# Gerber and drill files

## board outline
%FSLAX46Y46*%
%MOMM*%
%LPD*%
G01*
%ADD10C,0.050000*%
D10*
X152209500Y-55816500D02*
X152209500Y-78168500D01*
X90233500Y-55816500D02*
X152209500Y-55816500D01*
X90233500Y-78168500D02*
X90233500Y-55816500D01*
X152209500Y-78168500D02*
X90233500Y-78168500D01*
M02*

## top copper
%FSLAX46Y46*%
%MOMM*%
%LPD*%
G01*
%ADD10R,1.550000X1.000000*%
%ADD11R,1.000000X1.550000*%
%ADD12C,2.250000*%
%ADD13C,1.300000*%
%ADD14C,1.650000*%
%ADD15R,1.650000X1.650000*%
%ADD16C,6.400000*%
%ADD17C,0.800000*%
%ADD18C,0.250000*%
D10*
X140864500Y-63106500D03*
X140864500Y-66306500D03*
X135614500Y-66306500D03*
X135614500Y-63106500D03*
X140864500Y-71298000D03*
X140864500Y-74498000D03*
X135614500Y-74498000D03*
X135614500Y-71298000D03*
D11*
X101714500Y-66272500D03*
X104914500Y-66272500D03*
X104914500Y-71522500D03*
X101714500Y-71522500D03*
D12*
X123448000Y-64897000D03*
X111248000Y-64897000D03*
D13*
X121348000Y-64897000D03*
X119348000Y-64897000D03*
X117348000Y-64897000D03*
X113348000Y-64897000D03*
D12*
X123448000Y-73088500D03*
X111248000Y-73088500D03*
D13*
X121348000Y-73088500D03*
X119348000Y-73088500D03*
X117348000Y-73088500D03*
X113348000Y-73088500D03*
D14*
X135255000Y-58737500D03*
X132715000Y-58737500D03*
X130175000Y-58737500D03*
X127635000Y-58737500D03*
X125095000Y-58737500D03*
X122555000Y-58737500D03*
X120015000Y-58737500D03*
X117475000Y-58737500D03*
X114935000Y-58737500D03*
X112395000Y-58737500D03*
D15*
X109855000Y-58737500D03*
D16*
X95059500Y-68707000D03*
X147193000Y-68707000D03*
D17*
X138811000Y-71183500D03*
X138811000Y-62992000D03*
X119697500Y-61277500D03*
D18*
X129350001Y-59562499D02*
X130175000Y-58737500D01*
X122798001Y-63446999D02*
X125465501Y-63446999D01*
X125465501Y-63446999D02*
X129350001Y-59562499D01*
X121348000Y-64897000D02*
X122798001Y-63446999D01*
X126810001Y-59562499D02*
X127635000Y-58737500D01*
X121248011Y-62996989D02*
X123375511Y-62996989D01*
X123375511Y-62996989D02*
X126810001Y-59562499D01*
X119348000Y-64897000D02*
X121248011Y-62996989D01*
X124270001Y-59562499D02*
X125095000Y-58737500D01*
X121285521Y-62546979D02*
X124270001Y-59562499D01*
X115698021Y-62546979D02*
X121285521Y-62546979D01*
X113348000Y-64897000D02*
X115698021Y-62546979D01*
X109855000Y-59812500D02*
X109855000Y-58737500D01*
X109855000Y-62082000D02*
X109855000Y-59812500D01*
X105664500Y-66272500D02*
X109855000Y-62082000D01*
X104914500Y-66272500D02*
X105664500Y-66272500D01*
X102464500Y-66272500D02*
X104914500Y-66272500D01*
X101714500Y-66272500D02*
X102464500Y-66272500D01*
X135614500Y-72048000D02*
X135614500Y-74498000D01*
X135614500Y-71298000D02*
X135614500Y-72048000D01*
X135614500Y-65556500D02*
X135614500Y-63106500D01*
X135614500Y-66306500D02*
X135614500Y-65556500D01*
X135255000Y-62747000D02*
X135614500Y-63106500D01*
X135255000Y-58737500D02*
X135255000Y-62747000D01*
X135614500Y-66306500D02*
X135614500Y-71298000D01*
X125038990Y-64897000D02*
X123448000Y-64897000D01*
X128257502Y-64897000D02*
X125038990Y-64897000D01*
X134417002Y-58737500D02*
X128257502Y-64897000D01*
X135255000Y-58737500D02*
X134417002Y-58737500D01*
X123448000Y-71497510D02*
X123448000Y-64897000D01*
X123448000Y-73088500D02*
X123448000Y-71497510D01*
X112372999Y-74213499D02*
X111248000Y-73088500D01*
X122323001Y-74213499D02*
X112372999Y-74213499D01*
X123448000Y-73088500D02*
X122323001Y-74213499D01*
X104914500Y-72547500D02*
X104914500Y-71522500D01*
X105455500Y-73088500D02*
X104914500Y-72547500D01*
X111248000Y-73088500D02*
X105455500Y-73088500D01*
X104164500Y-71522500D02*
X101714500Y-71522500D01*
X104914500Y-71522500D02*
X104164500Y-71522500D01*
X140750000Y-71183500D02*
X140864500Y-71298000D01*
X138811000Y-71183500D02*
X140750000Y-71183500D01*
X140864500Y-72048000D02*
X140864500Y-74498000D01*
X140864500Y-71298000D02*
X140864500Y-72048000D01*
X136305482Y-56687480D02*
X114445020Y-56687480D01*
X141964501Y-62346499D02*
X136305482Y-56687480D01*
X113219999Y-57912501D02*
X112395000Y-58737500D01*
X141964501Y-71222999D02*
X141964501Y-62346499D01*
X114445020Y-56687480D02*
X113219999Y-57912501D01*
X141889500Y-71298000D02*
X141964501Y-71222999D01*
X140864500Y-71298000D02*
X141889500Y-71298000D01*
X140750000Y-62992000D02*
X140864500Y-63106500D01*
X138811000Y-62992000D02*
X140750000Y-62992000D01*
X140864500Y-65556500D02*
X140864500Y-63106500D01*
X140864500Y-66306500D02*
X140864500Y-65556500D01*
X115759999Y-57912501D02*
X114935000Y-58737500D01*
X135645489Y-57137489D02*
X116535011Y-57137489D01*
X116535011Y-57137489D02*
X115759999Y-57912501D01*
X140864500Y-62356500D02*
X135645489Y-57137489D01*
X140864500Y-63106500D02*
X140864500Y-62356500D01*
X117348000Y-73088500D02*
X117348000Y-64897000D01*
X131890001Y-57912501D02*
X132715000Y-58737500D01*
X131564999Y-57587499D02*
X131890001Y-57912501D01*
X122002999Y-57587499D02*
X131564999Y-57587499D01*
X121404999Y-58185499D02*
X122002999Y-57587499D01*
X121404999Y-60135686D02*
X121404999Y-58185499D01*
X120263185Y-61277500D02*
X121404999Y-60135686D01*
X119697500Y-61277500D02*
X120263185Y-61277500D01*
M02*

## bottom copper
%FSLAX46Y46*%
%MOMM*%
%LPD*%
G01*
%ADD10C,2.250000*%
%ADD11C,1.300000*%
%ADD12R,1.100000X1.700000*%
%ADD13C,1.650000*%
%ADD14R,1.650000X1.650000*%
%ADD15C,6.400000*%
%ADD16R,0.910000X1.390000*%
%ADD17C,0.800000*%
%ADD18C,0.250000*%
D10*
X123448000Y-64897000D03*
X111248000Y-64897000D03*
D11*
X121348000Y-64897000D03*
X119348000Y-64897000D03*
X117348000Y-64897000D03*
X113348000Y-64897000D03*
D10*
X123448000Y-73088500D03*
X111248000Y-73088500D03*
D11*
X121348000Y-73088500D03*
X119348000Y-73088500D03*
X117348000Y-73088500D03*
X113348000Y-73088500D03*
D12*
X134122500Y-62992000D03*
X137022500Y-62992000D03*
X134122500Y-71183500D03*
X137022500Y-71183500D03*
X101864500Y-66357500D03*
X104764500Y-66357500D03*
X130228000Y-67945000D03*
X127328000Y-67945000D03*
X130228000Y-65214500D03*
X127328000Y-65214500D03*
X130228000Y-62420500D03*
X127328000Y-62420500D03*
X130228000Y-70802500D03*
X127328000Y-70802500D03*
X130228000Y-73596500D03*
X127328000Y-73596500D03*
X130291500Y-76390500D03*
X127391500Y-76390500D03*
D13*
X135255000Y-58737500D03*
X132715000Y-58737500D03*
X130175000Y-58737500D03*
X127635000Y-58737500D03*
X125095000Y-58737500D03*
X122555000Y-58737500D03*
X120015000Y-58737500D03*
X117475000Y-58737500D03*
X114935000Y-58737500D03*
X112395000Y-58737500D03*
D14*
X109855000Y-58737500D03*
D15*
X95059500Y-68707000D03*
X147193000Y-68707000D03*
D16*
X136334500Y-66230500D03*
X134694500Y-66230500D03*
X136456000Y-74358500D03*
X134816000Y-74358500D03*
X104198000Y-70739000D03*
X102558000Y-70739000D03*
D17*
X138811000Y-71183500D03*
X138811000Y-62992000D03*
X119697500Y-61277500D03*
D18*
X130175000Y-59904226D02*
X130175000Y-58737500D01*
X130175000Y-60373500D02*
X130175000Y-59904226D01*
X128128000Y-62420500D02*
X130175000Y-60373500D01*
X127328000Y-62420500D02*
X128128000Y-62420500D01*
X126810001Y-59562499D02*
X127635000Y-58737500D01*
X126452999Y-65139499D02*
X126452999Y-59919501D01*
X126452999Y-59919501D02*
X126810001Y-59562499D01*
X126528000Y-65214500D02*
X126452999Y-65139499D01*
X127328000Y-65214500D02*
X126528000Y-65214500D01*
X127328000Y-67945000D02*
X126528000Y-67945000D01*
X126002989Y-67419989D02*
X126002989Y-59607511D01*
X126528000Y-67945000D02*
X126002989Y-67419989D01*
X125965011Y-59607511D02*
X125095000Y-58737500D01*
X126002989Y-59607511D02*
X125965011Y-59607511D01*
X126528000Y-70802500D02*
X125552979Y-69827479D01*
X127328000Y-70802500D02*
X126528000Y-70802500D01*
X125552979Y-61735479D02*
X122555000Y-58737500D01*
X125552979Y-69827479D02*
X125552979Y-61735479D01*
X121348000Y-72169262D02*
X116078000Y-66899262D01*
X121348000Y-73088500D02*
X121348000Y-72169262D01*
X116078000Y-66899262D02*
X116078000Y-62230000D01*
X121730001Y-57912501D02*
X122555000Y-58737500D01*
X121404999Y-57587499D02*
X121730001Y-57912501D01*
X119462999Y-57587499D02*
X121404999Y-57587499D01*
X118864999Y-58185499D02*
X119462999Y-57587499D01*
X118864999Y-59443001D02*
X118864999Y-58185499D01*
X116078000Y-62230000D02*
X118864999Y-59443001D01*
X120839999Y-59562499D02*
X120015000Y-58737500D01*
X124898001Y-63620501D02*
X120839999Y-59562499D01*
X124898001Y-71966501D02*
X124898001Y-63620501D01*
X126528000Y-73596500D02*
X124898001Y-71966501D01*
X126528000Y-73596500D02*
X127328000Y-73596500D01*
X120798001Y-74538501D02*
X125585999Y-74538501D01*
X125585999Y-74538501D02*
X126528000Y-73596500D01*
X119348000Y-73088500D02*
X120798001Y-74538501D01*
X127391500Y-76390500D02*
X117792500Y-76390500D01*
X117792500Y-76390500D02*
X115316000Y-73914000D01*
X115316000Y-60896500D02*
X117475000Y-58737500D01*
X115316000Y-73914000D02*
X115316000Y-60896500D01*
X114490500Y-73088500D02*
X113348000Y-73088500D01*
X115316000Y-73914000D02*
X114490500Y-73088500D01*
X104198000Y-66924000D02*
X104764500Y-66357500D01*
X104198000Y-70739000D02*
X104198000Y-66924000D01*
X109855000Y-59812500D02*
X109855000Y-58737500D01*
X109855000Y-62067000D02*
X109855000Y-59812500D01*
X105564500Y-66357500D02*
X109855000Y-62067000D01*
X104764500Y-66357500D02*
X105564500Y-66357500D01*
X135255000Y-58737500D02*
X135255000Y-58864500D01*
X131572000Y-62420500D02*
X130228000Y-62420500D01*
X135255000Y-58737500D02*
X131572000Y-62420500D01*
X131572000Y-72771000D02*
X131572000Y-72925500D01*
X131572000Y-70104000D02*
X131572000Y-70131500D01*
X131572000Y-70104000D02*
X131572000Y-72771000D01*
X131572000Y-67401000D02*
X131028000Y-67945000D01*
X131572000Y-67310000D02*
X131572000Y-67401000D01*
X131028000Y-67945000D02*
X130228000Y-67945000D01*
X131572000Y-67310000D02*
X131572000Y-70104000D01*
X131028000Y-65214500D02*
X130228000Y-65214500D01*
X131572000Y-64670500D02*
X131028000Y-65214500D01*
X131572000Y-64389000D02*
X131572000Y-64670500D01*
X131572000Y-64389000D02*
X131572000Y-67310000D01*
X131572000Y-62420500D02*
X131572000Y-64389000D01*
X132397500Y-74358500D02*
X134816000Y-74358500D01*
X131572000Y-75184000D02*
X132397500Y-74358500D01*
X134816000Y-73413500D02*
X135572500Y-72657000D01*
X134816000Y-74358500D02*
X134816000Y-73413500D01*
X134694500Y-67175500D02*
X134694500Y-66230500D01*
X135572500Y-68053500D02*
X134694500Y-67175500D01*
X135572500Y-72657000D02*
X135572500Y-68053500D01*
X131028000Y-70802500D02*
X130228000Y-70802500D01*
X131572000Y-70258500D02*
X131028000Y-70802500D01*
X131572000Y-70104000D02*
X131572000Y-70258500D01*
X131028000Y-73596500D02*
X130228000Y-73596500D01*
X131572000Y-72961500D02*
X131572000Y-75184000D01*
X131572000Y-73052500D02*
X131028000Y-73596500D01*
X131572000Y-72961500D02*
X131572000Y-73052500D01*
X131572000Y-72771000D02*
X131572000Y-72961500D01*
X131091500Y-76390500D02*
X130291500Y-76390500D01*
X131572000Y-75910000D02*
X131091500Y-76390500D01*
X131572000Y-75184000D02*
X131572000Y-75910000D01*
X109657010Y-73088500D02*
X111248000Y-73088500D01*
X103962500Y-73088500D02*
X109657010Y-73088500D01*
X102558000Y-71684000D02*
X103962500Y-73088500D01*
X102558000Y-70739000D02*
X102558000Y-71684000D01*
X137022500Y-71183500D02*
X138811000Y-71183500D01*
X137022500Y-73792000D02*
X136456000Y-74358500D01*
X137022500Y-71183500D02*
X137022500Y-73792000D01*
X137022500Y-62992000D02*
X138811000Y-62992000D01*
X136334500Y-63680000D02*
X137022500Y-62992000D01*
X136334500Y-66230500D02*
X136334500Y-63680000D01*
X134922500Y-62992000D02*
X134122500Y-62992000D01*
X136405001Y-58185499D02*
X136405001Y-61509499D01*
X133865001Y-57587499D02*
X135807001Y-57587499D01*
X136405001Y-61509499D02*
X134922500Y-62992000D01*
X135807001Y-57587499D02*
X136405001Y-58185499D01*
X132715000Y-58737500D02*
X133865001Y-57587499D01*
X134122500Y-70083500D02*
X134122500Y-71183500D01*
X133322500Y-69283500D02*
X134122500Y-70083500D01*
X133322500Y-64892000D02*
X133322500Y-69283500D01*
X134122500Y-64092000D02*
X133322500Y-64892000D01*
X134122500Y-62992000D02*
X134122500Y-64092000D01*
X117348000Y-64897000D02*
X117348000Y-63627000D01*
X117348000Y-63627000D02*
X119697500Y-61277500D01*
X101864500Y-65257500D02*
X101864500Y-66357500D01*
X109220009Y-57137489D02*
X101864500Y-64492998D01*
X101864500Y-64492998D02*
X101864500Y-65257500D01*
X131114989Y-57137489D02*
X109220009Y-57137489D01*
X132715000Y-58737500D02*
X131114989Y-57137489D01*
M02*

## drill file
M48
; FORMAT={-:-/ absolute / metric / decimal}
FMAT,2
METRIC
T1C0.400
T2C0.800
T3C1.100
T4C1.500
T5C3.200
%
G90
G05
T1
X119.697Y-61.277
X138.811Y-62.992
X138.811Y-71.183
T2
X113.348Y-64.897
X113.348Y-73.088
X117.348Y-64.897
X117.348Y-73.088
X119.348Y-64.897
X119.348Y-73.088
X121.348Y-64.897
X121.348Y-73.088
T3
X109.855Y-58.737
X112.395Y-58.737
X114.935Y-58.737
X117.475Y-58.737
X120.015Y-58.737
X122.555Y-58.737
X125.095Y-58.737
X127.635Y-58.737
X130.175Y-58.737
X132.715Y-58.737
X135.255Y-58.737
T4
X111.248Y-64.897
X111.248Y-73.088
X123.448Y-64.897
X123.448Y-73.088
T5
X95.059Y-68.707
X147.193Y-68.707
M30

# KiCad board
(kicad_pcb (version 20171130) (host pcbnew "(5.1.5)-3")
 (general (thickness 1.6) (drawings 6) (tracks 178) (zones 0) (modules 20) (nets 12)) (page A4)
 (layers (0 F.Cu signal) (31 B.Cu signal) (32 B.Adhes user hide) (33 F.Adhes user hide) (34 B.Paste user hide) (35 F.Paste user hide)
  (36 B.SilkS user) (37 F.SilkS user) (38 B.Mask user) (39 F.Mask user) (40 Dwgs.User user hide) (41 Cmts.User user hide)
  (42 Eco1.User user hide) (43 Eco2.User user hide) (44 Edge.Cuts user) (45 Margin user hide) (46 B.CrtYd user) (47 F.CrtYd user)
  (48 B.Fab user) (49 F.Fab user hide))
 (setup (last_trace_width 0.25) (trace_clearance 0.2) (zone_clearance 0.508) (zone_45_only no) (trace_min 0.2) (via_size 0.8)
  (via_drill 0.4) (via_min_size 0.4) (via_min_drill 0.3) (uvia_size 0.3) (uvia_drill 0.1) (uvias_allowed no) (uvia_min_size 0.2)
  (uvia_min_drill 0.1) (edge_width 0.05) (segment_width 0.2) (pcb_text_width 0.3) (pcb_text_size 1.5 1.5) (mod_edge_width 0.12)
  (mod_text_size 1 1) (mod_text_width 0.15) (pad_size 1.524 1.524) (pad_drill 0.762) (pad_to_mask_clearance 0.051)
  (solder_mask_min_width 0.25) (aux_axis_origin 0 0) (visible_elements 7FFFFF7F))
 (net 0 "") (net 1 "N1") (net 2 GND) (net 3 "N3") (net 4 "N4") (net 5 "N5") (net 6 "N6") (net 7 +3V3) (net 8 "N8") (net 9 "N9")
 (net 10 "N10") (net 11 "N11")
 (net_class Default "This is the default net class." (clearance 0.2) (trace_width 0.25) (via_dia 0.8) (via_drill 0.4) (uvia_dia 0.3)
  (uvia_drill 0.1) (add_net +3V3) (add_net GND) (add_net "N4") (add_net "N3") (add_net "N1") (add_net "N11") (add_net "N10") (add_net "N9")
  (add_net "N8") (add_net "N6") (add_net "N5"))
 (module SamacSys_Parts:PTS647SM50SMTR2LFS (layer F.Cu) (at 138.2395 64.7065)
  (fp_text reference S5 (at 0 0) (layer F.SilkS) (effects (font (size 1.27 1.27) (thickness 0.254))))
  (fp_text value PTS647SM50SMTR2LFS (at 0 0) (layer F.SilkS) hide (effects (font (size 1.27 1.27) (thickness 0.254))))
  (pad 4 smd rect (at 2.625 -1.6 90) (size 1 1.55) (layers F.Cu F.Paste F.Mask) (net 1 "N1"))
  (pad 3 smd rect (at 2.625 1.6 90) (size 1 1.55) (layers F.Cu F.Paste F.Mask) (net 1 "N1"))
  (pad 2 smd rect (at -2.625 1.6 90) (size 1 1.55) (layers F.Cu F.Paste F.Mask) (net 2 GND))
  (pad 1 smd rect (at -2.625 -1.6 90) (size 1 1.55) (layers F.Cu F.Paste F.Mask) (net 2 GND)))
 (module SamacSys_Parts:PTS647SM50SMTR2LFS (layer F.Cu) (at 138.2395 72.898)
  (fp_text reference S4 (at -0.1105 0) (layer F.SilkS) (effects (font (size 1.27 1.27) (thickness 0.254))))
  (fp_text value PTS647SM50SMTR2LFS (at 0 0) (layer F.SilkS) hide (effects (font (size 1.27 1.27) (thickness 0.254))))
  (pad 4 smd rect (at 2.625 -1.6 90) (size 1 1.55) (layers F.Cu F.Paste F.Mask) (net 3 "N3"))
  (pad 3 smd rect (at 2.625 1.6 90) (size 1 1.55) (layers F.Cu F.Paste F.Mask) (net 3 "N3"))
  (pad 2 smd rect (at -2.625 1.6 90) (size 1 1.55) (layers F.Cu F.Paste F.Mask) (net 2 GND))
  (pad 1 smd rect (at -2.625 -1.6 90) (size 1 1.55) (layers F.Cu F.Paste F.Mask) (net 2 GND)))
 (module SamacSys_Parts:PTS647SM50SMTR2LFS (layer F.Cu) (at 103.3145 68.8975 90)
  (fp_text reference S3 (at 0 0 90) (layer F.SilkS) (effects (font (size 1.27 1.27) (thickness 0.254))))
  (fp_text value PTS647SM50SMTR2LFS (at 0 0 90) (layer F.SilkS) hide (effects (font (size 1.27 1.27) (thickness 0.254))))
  (pad 4 smd rect (at 2.625 -1.6 180) (size 1 1.55) (layers F.Cu F.Paste F.Mask) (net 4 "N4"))
  (pad 3 smd rect (at 2.625 1.6 180) (size 1 1.55) (layers F.Cu F.Paste F.Mask) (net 4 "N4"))
  (pad 2 smd rect (at -2.625 1.6 180) (size 1 1.55) (layers F.Cu F.Paste F.Mask) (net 2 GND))
  (pad 1 smd rect (at -2.625 -1.6 180) (size 1 1.55) (layers F.Cu F.Paste F.Mask) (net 2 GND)))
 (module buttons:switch (layer F.Cu) (at 117.348 64.897)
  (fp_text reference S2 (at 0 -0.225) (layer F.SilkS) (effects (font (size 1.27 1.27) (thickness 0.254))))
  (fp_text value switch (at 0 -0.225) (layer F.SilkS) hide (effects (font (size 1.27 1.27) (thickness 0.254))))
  (pad 6 thru_hole circle (at 6.1 0) (size 2.25 2.25) (drill 1.5) (layers *.Cu *.Mask) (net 2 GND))
  (pad 5 thru_hole circle (at -6.1 0) (size 2.25 2.25) (drill 1.5) (layers *.Cu *.Mask) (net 2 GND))
  (pad 4 thru_hole circle (at 4 0) (size 1.3 1.3) (drill 0.8) (layers *.Cu *.Mask) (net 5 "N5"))
  (pad 3 thru_hole circle (at 2 0) (size 1.3 1.3) (drill 0.8) (layers *.Cu *.Mask) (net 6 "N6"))
  (pad 2 thru_hole circle (at 0 0) (size 1.3 1.3) (drill 0.8) (layers *.Cu *.Mask) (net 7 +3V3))
  (pad 1 thru_hole circle (at -4 0) (size 1.3 1.3) (drill 0.8) (layers *.Cu *.Mask) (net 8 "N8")))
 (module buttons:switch (layer F.Cu) (at 117.348 73.0885)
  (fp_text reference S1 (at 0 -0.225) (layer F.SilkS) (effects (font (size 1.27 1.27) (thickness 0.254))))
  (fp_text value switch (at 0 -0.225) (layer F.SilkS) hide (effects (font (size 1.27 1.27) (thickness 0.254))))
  (pad 6 thru_hole circle (at 6.1 0) (size 2.25 2.25) (drill 1.5) (layers *.Cu *.Mask) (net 2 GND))
  (pad 5 thru_hole circle (at -6.1 0) (size 2.25 2.25) (drill 1.5) (layers *.Cu *.Mask) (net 2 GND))
  (pad 4 thru_hole circle (at 4 0) (size 1.3 1.3) (drill 0.8) (layers *.Cu *.Mask) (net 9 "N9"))
  (pad 3 thru_hole circle (at 2 0) (size 1.3 1.3) (drill 0.8) (layers *.Cu *.Mask) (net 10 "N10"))
  (pad 2 thru_hole circle (at 0 0) (size 1.3 1.3) (drill 0.8) (layers *.Cu *.Mask) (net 7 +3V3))
  (pad 1 thru_hole circle (at -4 0) (size 1.3 1.3) (drill 0.8) (layers *.Cu *.Mask) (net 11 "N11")))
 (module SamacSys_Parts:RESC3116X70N (layer B.Cu) (at 135.5725 62.992 180)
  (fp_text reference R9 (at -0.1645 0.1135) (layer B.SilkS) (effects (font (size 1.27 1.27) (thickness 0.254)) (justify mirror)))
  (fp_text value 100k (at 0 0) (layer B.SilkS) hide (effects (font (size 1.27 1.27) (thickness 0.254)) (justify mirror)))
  (pad 2 smd rect (at 1.45 0 180) (size 1.1 1.7) (layers B.Cu B.Paste B.Mask) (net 7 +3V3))
  (pad 1 smd rect (at -1.45 0 180) (size 1.1 1.7) (layers B.Cu B.Paste B.Mask) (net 1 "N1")))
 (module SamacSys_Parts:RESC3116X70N (layer B.Cu) (at 135.5725 71.1835 180)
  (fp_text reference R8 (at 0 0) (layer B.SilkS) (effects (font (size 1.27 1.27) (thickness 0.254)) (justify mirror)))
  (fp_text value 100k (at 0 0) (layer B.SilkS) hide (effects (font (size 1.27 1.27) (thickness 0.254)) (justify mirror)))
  (pad 2 smd rect (at 1.45 0 180) (size 1.1 1.7) (layers B.Cu B.Paste B.Mask) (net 7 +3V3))
  (pad 1 smd rect (at -1.45 0 180) (size 1.1 1.7) (layers B.Cu B.Paste B.Mask) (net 3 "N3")))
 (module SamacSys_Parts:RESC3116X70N (layer B.Cu) (at 103.3145 66.3575 180)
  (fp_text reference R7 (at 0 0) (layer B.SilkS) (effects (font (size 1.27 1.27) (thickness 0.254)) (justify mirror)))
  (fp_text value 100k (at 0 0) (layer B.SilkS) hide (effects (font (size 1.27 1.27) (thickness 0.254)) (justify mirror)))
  (pad 2 smd rect (at 1.45 0 180) (size 1.1 1.7) (layers B.Cu B.Paste B.Mask) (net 7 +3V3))
  (pad 1 smd rect (at -1.45 0 180) (size 1.1 1.7) (layers B.Cu B.Paste B.Mask) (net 4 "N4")))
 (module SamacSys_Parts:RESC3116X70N (layer B.Cu) (at 128.778 67.945)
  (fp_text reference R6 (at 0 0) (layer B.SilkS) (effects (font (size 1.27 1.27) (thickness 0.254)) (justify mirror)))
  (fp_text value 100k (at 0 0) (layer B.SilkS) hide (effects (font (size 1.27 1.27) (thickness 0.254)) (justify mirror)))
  (pad 2 smd rect (at 1.45 0) (size 1.1 1.7) (layers B.Cu B.Paste B.Mask) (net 2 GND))
  (pad 1 smd rect (at -1.45 0) (size 1.1 1.7) (layers B.Cu B.Paste B.Mask) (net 8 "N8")))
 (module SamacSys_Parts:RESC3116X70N (layer B.Cu) (at 128.778 65.2145)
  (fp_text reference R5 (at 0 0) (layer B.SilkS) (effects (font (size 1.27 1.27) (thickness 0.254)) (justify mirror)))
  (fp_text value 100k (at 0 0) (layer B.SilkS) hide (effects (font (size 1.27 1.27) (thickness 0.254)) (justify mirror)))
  (pad 2 smd rect (at 1.45 0) (size 1.1 1.7) (layers B.Cu B.Paste B.Mask) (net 2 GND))
  (pad 1 smd rect (at -1.45 0) (size 1.1 1.7) (layers B.Cu B.Paste B.Mask) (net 6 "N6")))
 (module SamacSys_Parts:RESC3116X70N (layer B.Cu) (at 128.778 62.4205)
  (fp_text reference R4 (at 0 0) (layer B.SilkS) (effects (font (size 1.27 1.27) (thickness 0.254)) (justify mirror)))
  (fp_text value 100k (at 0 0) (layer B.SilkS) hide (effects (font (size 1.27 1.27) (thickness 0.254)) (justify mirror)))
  (pad 2 smd rect (at 1.45 0) (size 1.1 1.7) (layers B.Cu B.Paste B.Mask) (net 2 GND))
  (pad 1 smd rect (at -1.45 0) (size 1.1 1.7) (layers B.Cu B.Paste B.Mask) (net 5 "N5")))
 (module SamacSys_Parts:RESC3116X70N (layer B.Cu) (at 128.778 70.8025)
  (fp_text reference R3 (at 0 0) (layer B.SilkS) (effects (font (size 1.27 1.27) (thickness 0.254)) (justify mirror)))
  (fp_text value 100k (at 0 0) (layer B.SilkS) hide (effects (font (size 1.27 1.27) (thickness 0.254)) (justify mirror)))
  (pad 2 smd rect (at 1.45 0) (size 1.1 1.7) (layers B.Cu B.Paste B.Mask) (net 2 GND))
  (pad 1 smd rect (at -1.45 0) (size 1.1 1.7) (layers B.Cu B.Paste B.Mask) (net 9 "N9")))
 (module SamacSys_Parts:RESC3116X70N (layer B.Cu) (at 128.778 73.5965)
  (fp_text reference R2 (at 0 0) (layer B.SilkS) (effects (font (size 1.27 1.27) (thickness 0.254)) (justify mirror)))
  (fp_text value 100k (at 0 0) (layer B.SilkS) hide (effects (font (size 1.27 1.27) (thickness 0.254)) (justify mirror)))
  (pad 2 smd rect (at 1.45 0) (size 1.1 1.7) (layers B.Cu B.Paste B.Mask) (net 2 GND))
  (pad 1 smd rect (at -1.45 0) (size 1.1 1.7) (layers B.Cu B.Paste B.Mask) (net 10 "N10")))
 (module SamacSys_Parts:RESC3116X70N (layer B.Cu) (at 128.8415 76.3905)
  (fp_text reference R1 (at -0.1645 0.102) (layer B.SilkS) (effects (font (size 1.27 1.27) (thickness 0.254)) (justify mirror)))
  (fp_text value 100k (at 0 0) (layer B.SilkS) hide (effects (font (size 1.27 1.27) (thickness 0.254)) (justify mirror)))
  (pad 2 smd rect (at 1.45 0) (size 1.1 1.7) (layers B.Cu B.Paste B.Mask) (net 2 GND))
  (pad 1 smd rect (at -1.45 0) (size 1.1 1.7) (layers B.Cu B.Paste B.Mask) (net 11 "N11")))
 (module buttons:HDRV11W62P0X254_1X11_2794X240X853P (layer F.Cu) (at 109.855 58.7375)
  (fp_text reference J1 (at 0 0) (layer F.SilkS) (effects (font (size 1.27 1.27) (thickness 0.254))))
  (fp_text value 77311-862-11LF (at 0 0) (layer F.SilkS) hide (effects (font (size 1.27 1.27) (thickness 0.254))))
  (pad 11 thru_hole circle (at 25.4 0) (size 1.65 1.65) (drill 1.1) (layers *.Cu *.Mask) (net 2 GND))
  (pad 10 thru_hole circle (at 22.86 0) (size 1.65 1.65) (drill 1.1) (layers *.Cu *.Mask) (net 7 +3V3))
  (pad 9 thru_hole circle (at 20.32 0) (size 1.65 1.65) (drill 1.1) (layers *.Cu *.Mask) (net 5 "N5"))
  (pad 8 thru_hole circle (at 17.78 0) (size 1.65 1.65) (drill 1.1) (layers *.Cu *.Mask) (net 6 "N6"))
  (pad 7 thru_hole circle (at 15.24 0) (size 1.65 1.65) (drill 1.1) (layers *.Cu *.Mask) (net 8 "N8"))
  (pad 6 thru_hole circle (at 12.7 0) (size 1.65 1.65) (drill 1.1) (layers *.Cu *.Mask) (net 9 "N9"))
  (pad 5 thru_hole circle (at 10.16 0) (size 1.65 1.65) (drill 1.1) (layers *.Cu *.Mask) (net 10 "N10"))
  (pad 4 thru_hole circle (at 7.62 0) (size 1.65 1.65) (drill 1.1) (layers *.Cu *.Mask) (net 11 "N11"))
  (pad 3 thru_hole circle (at 5.08 0) (size 1.65 1.65) (drill 1.1) (layers *.Cu *.Mask) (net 1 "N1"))
  (pad 2 thru_hole circle (at 2.54 0) (size 1.65 1.65) (drill 1.1) (layers *.Cu *.Mask) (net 3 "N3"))
  (pad 1 thru_hole rect (at 0 0) (size 1.65 1.65) (drill 1.1) (layers *.Cu *.Mask) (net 4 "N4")))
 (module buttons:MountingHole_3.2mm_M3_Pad (layer F.Cu) (at 95.0595 68.707)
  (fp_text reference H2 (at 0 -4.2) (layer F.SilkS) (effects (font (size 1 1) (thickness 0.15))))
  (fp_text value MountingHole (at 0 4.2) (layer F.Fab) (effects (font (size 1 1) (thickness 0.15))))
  (pad 1 thru_hole circle (at 0 0) (size 6.4 6.4) (drill 3.2) (layers *.Cu *.Mask)))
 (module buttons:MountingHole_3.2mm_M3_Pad (layer F.Cu) (at 147.193 68.707)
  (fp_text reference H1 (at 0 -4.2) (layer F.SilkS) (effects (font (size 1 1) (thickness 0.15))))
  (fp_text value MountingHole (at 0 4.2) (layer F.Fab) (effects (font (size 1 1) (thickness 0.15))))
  (pad 1 thru_hole circle (at 0 0) (size 6.4 6.4) (drill 3.2) (layers *.Cu *.Mask)))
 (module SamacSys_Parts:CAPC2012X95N (layer B.Cu) (at 135.5145 66.2305)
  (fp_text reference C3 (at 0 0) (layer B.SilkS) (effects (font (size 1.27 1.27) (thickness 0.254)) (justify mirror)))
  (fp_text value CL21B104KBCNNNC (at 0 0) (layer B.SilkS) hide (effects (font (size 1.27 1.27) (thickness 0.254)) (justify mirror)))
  (pad 2 smd rect (at 0.82 0) (size 0.91 1.39) (layers B.Cu B.Paste B.Mask) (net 1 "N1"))
  (pad 1 smd rect (at -0.82 0) (size 0.91 1.39) (layers B.Cu B.Paste B.Mask) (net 2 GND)))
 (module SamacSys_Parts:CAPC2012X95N (layer B.Cu) (at 135.636 74.3585)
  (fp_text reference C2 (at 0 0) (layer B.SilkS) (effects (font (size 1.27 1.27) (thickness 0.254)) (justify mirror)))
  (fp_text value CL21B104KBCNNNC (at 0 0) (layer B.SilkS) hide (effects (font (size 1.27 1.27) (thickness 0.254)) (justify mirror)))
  (pad 2 smd rect (at 0.82 0) (size 0.91 1.39) (layers B.Cu B.Paste B.Mask) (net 3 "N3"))
  (pad 1 smd rect (at -0.82 0) (size 0.91 1.39) (layers B.Cu B.Paste B.Mask) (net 2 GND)))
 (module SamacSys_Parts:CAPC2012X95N (layer B.Cu) (at 103.378 70.739)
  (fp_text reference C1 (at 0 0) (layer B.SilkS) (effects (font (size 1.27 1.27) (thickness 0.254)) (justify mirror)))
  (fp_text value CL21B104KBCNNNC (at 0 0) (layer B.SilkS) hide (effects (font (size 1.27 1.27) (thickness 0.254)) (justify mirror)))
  (pad 2 smd rect (at 0.82 0) (size 0.91 1.39) (layers B.Cu B.Paste B.Mask) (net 4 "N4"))
  (pad 1 smd rect (at -0.82 0) (size 0.91 1.39) (layers B.Cu B.Paste B.Mask) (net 2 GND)))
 (gr_line (start 152.2095 55.8165) (end 152.2095 78.1685) (layer Edge.Cuts) (width 0.05))
 (gr_line (start 90.2335 55.8165) (end 152.2095 55.8165) (layer Edge.Cuts) (width 0.05))
 (gr_line (start 90.2335 78.1685) (end 90.2335 55.8165) (layer Edge.Cuts) (width 0.05))
 (gr_line (start 152.2095 78.1685) (end 90.2335 78.1685) (layer Edge.Cuts) (width 0.05))
 (segment (start 130.175 59.904226) (end 130.175 58.7375) (width 0.25) (layer B.Cu) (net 5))
 (segment (start 130.175 60.3735) (end 130.175 59.904226) (width 0.25) (layer B.Cu) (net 5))
 (segment (start 128.128 62.4205) (end 130.175 60.3735) (width 0.25) (layer B.Cu) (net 5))
 (segment (start 127.328 62.4205) (end 128.128 62.4205) (width 0.25) (layer B.Cu) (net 5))
 (segment (start 129.350001 59.562499) (end 130.175 58.7375) (width 0.25) (layer F.Cu) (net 5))
 (segment (start 122.798001 63.446999) (end 125.465501 63.446999) (width 0.25) (layer F.Cu) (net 5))
 (segment (start 125.465501 63.446999) (end 129.350001 59.562499) (width 0.25) (layer F.Cu) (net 5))
 (segment (start 121.348 64.897) (end 122.798001 63.446999) (width 0.25) (layer F.Cu) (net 5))
 (segment (start 126.810001 59.562499) (end 127.635 58.7375) (width 0.25) (layer B.Cu) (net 6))
 (segment (start 126.452999 65.139499) (end 126.452999 59.919501) (width 0.25) (layer B.Cu) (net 6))
 (segment (start 126.452999 59.919501) (end 126.810001 59.562499) (width 0.25) (layer B.Cu) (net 6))
 (segment (start 126.528 65.2145) (end 126.452999 65.139499) (width 0.25) (layer B.Cu) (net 6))
 (segment (start 127.328 65.2145) (end 126.528 65.2145) (width 0.25) (layer B.Cu) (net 6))
 (segment (start 126.810001 59.562499) (end 127.635 58.7375) (width 0.25) (layer F.Cu) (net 6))
 (segment (start 121.248011 62.996989) (end 123.375511 62.996989) (width 0.25) (layer F.Cu) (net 6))
 (segment (start 123.375511 62.996989) (end 126.810001 59.562499) (width 0.25) (layer F.Cu) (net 6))
 (segment (start 119.348 64.897) (end 121.248011 62.996989) (width 0.25) (layer F.Cu) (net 6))
 (segment (start 127.328 67.945) (end 126.528 67.945) (width 0.25) (layer B.Cu) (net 8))
 (segment (start 126.002989 67.419989) (end 126.002989 59.607511) (width 0.25) (layer B.Cu) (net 8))
 (segment (start 126.528 67.945) (end 126.002989 67.419989) (width 0.25) (layer B.Cu) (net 8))
 (segment (start 125.965011 59.607511) (end 125.095 58.7375) (width 0.25) (layer B.Cu) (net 8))
 (segment (start 126.002989 59.607511) (end 125.965011 59.607511) (width 0.25) (layer B.Cu) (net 8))
 (segment (start 124.270001 59.562499) (end 125.095 58.7375) (width 0.25) (layer F.Cu) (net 8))
 (segment (start 121.285521 62.546979) (end 124.270001 59.562499) (width 0.25) (layer F.Cu) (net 8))
 (segment (start 115.698021 62.546979) (end 121.285521 62.546979) (width 0.25) (layer F.Cu) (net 8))
 (segment (start 113.348 64.897) (end 115.698021 62.546979) (width 0.25) (layer F.Cu) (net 8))
 (segment (start 126.528 70.8025) (end 125.552979 69.827479) (width 0.25) (layer B.Cu) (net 9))
 (segment (start 127.328 70.8025) (end 126.528 70.8025) (width 0.25) (layer B.Cu) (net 9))
 (segment (start 125.552979 61.735479) (end 122.555 58.7375) (width 0.25) (layer B.Cu) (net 9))
 (segment (start 125.552979 69.827479) (end 125.552979 61.735479) (width 0.25) (layer B.Cu) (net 9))
 (segment (start 121.348 72.169262) (end 116.078 66.899262) (width 0.25) (layer B.Cu) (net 9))
 (segment (start 121.348 73.0885) (end 121.348 72.169262) (width 0.25) (layer B.Cu) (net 9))
 (segment (start 116.078 66.899262) (end 116.078 62.23) (width 0.25) (layer B.Cu) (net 9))
 (segment (start 121.730001 57.912501) (end 122.555 58.7375) (width 0.25) (layer B.Cu) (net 9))
 (segment (start 121.404999 57.587499) (end 121.730001 57.912501) (width 0.25) (layer B.Cu) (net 9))
 (segment (start 119.462999 57.587499) (end 121.404999 57.587499) (width 0.25) (layer B.Cu) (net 9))
 (segment (start 118.864999 58.185499) (end 119.462999 57.587499) (width 0.25) (layer B.Cu) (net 9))
 (segment (start 118.864999 59.443001) (end 118.864999 58.185499) (width 0.25) (layer B.Cu) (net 9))
 (segment (start 116.078 62.23) (end 118.864999 59.443001) (width 0.25) (layer B.Cu) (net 9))
 (segment (start 120.839999 59.562499) (end 120.015 58.7375) (width 0.25) (layer B.Cu) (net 10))
 (segment (start 124.898001 63.620501) (end 120.839999 59.562499) (width 0.25) (layer B.Cu) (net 10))
 (segment (start 124.898001 71.966501) (end 124.898001 63.620501) (width 0.25) (layer B.Cu) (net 10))
 (segment (start 126.528 73.5965) (end 124.898001 71.966501) (width 0.25) (layer B.Cu) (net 10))
 (segment (start 126.528 73.5965) (end 127.328 73.5965) (width 0.25) (layer B.Cu) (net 10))
 (segment (start 120.798001 74.538501) (end 125.585999 74.538501) (width 0.25) (layer B.Cu) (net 10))
 (segment (start 125.585999 74.538501) (end 126.528 73.5965) (width 0.25) (layer B.Cu) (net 10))
 (segment (start 119.348 73.0885) (end 120.798001 74.538501) (width 0.25) (layer B.Cu) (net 10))
 (segment (start 127.3915 76.3905) (end 117.7925 76.3905) (width 0.25) (layer B.Cu) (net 11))
 (segment (start 117.7925 76.3905) (end 115.316 73.914) (width 0.25) (layer B.Cu) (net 11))
 (segment (start 115.316 60.8965) (end 117.475 58.7375) (width 0.25) (layer B.Cu) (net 11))
 (segment (start 115.316 73.914) (end 115.316 60.8965) (width 0.25) (layer B.Cu) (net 11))
 (segment (start 114.4905 73.0885) (end 113.348 73.0885) (width 0.25) (layer B.Cu) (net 11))
 (segment (start 115.316 73.914) (end 114.4905 73.0885) (width 0.25) (layer B.Cu) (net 11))
 (segment (start 104.198 66.924) (end 104.7645 66.3575) (width 0.25) (layer B.Cu) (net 4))
 (segment (start 104.198 70.739) (end 104.198 66.924) (width 0.25) (layer B.Cu) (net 4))
 (segment (start 109.855 59.8125) (end 109.855 58.7375) (width 0.25) (layer B.Cu) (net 4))
 (segment (start 109.855 62.067) (end 109.855 59.8125) (width 0.25) (layer B.Cu) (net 4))
 (segment (start 105.5645 66.3575) (end 109.855 62.067) (width 0.25) (layer B.Cu) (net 4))
 (segment (start 104.7645 66.3575) (end 105.5645 66.3575) (width 0.25) (layer B.Cu) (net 4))
 (segment (start 109.855 59.8125) (end 109.855 58.7375) (width 0.25) (layer F.Cu) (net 4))
 (segment (start 109.855 62.082) (end 109.855 59.8125) (width 0.25) (layer F.Cu) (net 4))
 (segment (start 105.6645 66.2725) (end 109.855 62.082) (width 0.25) (layer F.Cu) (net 4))
 (segment (start 104.9145 66.2725) (end 105.6645 66.2725) (width 0.25) (layer F.Cu) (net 4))
 (segment (start 102.4645 66.2725) (end 104.9145 66.2725) (width 0.25) (layer F.Cu) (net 4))
 (segment (start 101.7145 66.2725) (end 102.4645 66.2725) (width 0.25) (layer F.Cu) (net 4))
 (segment (start 135.255 58.7375) (end 135.255 58.8645) (width 0.25) (layer B.Cu) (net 2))
 (segment (start 131.572 62.4205) (end 130.228 62.4205) (width 0.25) (layer B.Cu) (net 2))
 (segment (start 135.255 58.7375) (end 131.572 62.4205) (width 0.25) (layer B.Cu) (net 2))
 (segment (start 131.572 72.771) (end 131.572 72.9255) (width 0.25) (layer B.Cu) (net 2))
 (segment (start 131.572 70.104) (end 131.572 70.1315) (width 0.25) (layer B.Cu) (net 2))
 (segment (start 131.572 70.104) (end 131.572 72.771) (width 0.25) (layer B.Cu) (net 2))
 (segment (start 131.572 67.401) (end 131.028 67.945) (width 0.25) (layer B.Cu) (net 2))
 (segment (start 131.572 67.31) (end 131.572 67.401) (width 0.25) (layer B.Cu) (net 2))
 (segment (start 131.028 67.945) (end 130.228 67.945) (width 0.25) (layer B.Cu) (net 2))
 (segment (start 131.572 67.31) (end 131.572 70.104) (width 0.25) (layer B.Cu) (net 2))
 (segment (start 131.028 65.2145) (end 130.228 65.2145) (width 0.25) (layer B.Cu) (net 2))
 (segment (start 131.572 64.6705) (end 131.028 65.2145) (width 0.25) (layer B.Cu) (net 2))
 (segment (start 131.572 64.389) (end 131.572 64.6705) (width 0.25) (layer B.Cu) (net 2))
 (segment (start 131.572 64.389) (end 131.572 67.31) (width 0.25) (layer B.Cu) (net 2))
 (segment (start 131.572 62.4205) (end 131.572 64.389) (width 0.25) (layer B.Cu) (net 2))
 (segment (start 135.6145 72.048) (end 135.6145 74.498) (width 0.25) (layer F.Cu) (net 2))
 (segment (start 135.6145 71.298) (end 135.6145 72.048) (width 0.25) (layer F.Cu) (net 2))
 (segment (start 135.6145 65.5565) (end 135.6145 63.1065) (width 0.25) (layer F.Cu) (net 2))
 (segment (start 135.6145 66.3065) (end 135.6145 65.5565) (width 0.25) (layer F.Cu) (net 2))
 (segment (start 132.3975 74.3585) (end 134.816 74.3585) (width 0.25) (layer B.Cu) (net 2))
 (segment (start 131.572 75.184) (end 132.3975 74.3585) (width 0.25) (layer B.Cu) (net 2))
 (segment (start 134.816 73.4135) (end 135.5725 72.657) (width 0.25) (layer B.Cu) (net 2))
 (segment (start 134.816 74.3585) (end 134.816 73.4135) (width 0.25) (layer B.Cu) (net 2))
 (segment (start 134.6945 67.1755) (end 134.6945 66.2305) (width 0.25) (layer B.Cu) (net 2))
 (segment (start 135.5725 68.0535) (end 134.6945 67.1755) (width 0.25) (layer B.Cu) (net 2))
 (segment (start 135.5725 72.657) (end 135.5725 68.0535) (width 0.25) (layer B.Cu) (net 2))
 (segment (start 135.255 62.747) (end 135.6145 63.1065) (width 0.25) (layer F.Cu) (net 2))
 (segment (start 135.255 58.7375) (end 135.255 62.747) (width 0.25) (layer F.Cu) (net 2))
 (segment (start 135.6145 66.3065) (end 135.6145 71.298) (width 0.25) (layer F.Cu) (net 2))
 (segment (start 131.028 70.8025) (end 130.228 70.8025) (width 0.25) (layer B.Cu) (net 2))
 (segment (start 131.572 70.2585) (end 131.028 70.8025) (width 0.25) (layer B.Cu) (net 2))
 (segment (start 131.572 70.104) (end 131.572 70.2585) (width 0.25) (layer B.Cu) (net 2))
 (segment (start 131.028 73.5965) (end 130.228 73.5965) (width 0.25) (layer B.Cu) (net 2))
 (segment (start 131.572 72.9615) (end 131.572 75.184) (width 0.25) (layer B.Cu) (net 2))
 (segment (start 131.572 73.0525) (end 131.028 73.5965) (width 0.25) (layer B.Cu) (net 2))
 (segment (start 131.572 72.9615) (end 131.572 73.0525) (width 0.25) (layer B.Cu) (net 2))
 (segment (start 131.572 72.771) (end 131.572 72.9615) (width 0.25) (layer B.Cu) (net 2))
 (segment (start 131.0915 76.3905) (end 130.2915 76.3905) (width 0.25) (layer B.Cu) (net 2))
 (segment (start 131.572 75.91) (end 131.0915 76.3905) (width 0.25) (layer B.Cu) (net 2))
 (segment (start 131.572 75.184) (end 131.572 75.91) (width 0.25) (layer B.Cu) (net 2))
 (segment (start 125.03899 64.897) (end 123.448 64.897) (width 0.25) (layer F.Cu) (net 2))
 (segment (start 128.257502 64.897) (end 125.03899 64.897) (width 0.25) (layer F.Cu) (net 2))
 (segment (start 134.417002 58.7375) (end 128.257502 64.897) (width 0.25) (layer F.Cu) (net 2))
 (segment (start 135.255 58.7375) (end 134.417002 58.7375) (width 0.25) (layer F.Cu) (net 2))
 (segment (start 123.448 71.49751) (end 123.448 64.897) (width 0.25) (layer F.Cu) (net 2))
 (segment (start 123.448 73.0885) (end 123.448 71.49751) (width 0.25) (layer F.Cu) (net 2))
 (segment (start 112.372999 74.213499) (end 111.248 73.0885) (width 0.25) (layer F.Cu) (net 2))
 (segment (start 122.323001 74.213499) (end 112.372999 74.213499) (width 0.25) (layer F.Cu) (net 2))
 (segment (start 123.448 73.0885) (end 122.323001 74.213499) (width 0.25) (layer F.Cu) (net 2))
 (segment (start 104.9145 72.5475) (end 104.9145 71.5225) (width 0.25) (layer F.Cu) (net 2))
 (segment (start 105.4555 73.0885) (end 104.9145 72.5475) (width 0.25) (layer F.Cu) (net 2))
 (segment (start 111.248 73.0885) (end 105.4555 73.0885) (width 0.25) (layer F.Cu) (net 2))
 (segment (start 104.1645 71.5225) (end 101.7145 71.5225) (width 0.25) (layer F.Cu) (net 2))
 (segment (start 104.9145 71.5225) (end 104.1645 71.5225) (width 0.25) (layer F.Cu) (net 2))
 (segment (start 109.65701 73.0885) (end 111.248 73.0885) (width 0.25) (layer B.Cu) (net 2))
 (segment (start 103.9625 73.0885) (end 109.65701 73.0885) (width 0.25) (layer B.Cu) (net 2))
 (segment (start 102.558 71.684) (end 103.9625 73.0885) (width 0.25) (layer B.Cu) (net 2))
 (segment (start 102.558 70.739) (end 102.558 71.684) (width 0.25) (layer B.Cu) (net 2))
 (via (at 138.811 71.1835) (size 0.8) (drill 0.4) (layers F.Cu B.Cu) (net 3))
 (segment (start 137.0225 71.1835) (end 138.811 71.1835) (width 0.25) (layer B.Cu) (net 3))
 (segment (start 140.75 71.1835) (end 140.8645 71.298) (width 0.25) (layer F.Cu) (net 3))
 (segment (start 138.811 71.1835) (end 140.75 71.1835) (width 0.25) (layer F.Cu) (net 3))
 (segment (start 140.8645 72.048) (end 140.8645 74.498) (width 0.25) (layer F.Cu) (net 3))
 (segment (start 140.8645 71.298) (end 140.8645 72.048) (width 0.25) (layer F.Cu) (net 3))
 (segment (start 137.0225 73.792) (end 136.456 74.3585) (width 0.25) (layer B.Cu) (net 3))
 (segment (start 137.0225 71.1835) (end 137.0225 73.792) (width 0.25) (layer B.Cu) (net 3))
 (segment (start 136.305482 56.68748) (end 114.44502 56.68748) (width 0.25) (layer F.Cu) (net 3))
 (segment (start 141.964501 62.346499) (end 136.305482 56.68748) (width 0.25) (layer F.Cu) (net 3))
 (segment (start 113.219999 57.912501) (end 112.395 58.7375) (width 0.25) (layer F.Cu) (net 3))
 (segment (start 141.964501 71.222999) (end 141.964501 62.346499) (width 0.25) (layer F.Cu) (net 3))
 (segment (start 114.44502 56.68748) (end 113.219999 57.912501) (width 0.25) (layer F.Cu) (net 3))
 (segment (start 141.8895 71.298) (end 141.964501 71.222999) (width 0.25) (layer F.Cu) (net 3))
 (segment (start 140.8645 71.298) (end 141.8895 71.298) (width 0.25) (layer F.Cu) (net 3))
 (via (at 138.811 62.992) (size 0.8) (drill 0.4) (layers F.Cu B.Cu) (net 1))
 (segment (start 137.0225 62.992) (end 138.811 62.992) (width 0.25) (layer B.Cu) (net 1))
 (segment (start 140.75 62.992) (end 140.8645 63.1065) (width 0.25) (layer F.Cu) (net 1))
 (segment (start 138.811 62.992) (end 140.75 62.992) (width 0.25) (layer F.Cu) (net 1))
 (segment (start 140.8645 65.5565) (end 140.8645 63.1065) (width 0.25) (layer F.Cu) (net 1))
 (segment (start 140.8645 66.3065) (end 140.8645 65.5565) (width 0.25) (layer F.Cu) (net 1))
 (segment (start 136.3345 63.68) (end 137.0225 62.992) (width 0.25) (layer B.Cu) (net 1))
 (segment (start 136.3345 66.2305) (end 136.3345 63.68) (width 0.25) (layer B.Cu) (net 1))
 (segment (start 115.759999 57.912501) (end 114.935 58.7375) (width 0.25) (layer F.Cu) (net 1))
 (segment (start 135.645489 57.137489) (end 116.535011 57.137489) (width 0.25) (layer F.Cu) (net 1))
 (segment (start 116.535011 57.137489) (end 115.759999 57.912501) (width 0.25) (layer F.Cu) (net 1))
 (segment (start 140.8645 62.3565) (end 135.645489 57.137489) (width 0.25) (layer F.Cu) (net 1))
 (segment (start 140.8645 63.1065) (end 140.8645 62.3565) (width 0.25) (layer F.Cu) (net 1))
 (segment (start 134.9225 62.992) (end 134.1225 62.992) (width 0.25) (layer B.Cu) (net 7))
 (segment (start 136.405001 58.185499) (end 136.405001 61.509499) (width 0.25) (layer B.Cu) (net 7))
 (segment (start 133.865001 57.587499) (end 135.807001 57.587499) (width 0.25) (layer B.Cu) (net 7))
 (segment (start 136.405001 61.509499) (end 134.9225 62.992) (width 0.25) (layer B.Cu) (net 7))
 (segment (start 135.807001 57.587499) (end 136.405001 58.185499) (width 0.25) (layer B.Cu) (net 7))
 (segment (start 132.715 58.7375) (end 133.865001 57.587499) (width 0.25) (layer B.Cu) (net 7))
 (segment (start 134.1225 70.0835) (end 134.1225 71.1835) (width 0.25) (layer B.Cu) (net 7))
 (segment (start 133.3225 69.2835) (end 134.1225 70.0835) (width 0.25) (layer B.Cu) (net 7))
 (segment (start 133.3225 64.892) (end 133.3225 69.2835) (width 0.25) (layer B.Cu) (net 7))
 (segment (start 134.1225 64.092) (end 133.3225 64.892) (width 0.25) (layer B.Cu) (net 7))
 (segment (start 134.1225 62.992) (end 134.1225 64.092) (width 0.25) (layer B.Cu) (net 7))
 (segment (start 117.348 73.0885) (end 117.348 64.897) (width 0.25) (layer F.Cu) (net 7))
 (via (at 119.6975 61.2775) (size 0.8) (drill 0.4) (layers F.Cu B.Cu) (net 7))
 (segment (start 117.348 64.897) (end 117.348 63.627) (width 0.25) (layer B.Cu) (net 7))
 (segment (start 117.348 63.627) (end 119.6975 61.2775) (width 0.25) (layer B.Cu) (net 7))
 (segment (start 131.890001 57.912501) (end 132.715 58.7375) (width 0.25) (layer F.Cu) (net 7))
 (segment (start 131.564999 57.587499) (end 131.890001 57.912501) (width 0.25) (layer F.Cu) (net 7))
 (segment (start 122.002999 57.587499) (end 131.564999 57.587499) (width 0.25) (layer F.Cu) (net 7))
 (segment (start 121.404999 58.185499) (end 122.002999 57.587499) (width 0.25) (layer F.Cu) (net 7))
 (segment (start 121.404999 60.135686) (end 121.404999 58.185499) (width 0.25) (layer F.Cu) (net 7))
 (segment (start 120.263185 61.2775) (end 121.404999 60.135686) (width 0.25) (layer F.Cu) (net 7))
 (segment (start 119.6975 61.2775) (end 120.263185 61.2775) (width 0.25) (layer F.Cu) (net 7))
 (segment (start 101.8645 65.2575) (end 101.8645 66.3575) (width 0.25) (layer B.Cu) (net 7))
 (segment (start 109.220009 57.137489) (end 101.8645 64.492998) (width 0.25) (layer B.Cu) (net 7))
 (segment (start 101.8645 64.492998) (end 101.8645 65.2575) (width 0.25) (layer B.Cu) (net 7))
 (segment (start 131.114989 57.137489) (end 109.220009 57.137489) (width 0.25) (layer B.Cu) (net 7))
 (segment (start 132.715 58.7375) (end 131.114989 57.137489) (width 0.25) (layer B.Cu) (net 7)))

